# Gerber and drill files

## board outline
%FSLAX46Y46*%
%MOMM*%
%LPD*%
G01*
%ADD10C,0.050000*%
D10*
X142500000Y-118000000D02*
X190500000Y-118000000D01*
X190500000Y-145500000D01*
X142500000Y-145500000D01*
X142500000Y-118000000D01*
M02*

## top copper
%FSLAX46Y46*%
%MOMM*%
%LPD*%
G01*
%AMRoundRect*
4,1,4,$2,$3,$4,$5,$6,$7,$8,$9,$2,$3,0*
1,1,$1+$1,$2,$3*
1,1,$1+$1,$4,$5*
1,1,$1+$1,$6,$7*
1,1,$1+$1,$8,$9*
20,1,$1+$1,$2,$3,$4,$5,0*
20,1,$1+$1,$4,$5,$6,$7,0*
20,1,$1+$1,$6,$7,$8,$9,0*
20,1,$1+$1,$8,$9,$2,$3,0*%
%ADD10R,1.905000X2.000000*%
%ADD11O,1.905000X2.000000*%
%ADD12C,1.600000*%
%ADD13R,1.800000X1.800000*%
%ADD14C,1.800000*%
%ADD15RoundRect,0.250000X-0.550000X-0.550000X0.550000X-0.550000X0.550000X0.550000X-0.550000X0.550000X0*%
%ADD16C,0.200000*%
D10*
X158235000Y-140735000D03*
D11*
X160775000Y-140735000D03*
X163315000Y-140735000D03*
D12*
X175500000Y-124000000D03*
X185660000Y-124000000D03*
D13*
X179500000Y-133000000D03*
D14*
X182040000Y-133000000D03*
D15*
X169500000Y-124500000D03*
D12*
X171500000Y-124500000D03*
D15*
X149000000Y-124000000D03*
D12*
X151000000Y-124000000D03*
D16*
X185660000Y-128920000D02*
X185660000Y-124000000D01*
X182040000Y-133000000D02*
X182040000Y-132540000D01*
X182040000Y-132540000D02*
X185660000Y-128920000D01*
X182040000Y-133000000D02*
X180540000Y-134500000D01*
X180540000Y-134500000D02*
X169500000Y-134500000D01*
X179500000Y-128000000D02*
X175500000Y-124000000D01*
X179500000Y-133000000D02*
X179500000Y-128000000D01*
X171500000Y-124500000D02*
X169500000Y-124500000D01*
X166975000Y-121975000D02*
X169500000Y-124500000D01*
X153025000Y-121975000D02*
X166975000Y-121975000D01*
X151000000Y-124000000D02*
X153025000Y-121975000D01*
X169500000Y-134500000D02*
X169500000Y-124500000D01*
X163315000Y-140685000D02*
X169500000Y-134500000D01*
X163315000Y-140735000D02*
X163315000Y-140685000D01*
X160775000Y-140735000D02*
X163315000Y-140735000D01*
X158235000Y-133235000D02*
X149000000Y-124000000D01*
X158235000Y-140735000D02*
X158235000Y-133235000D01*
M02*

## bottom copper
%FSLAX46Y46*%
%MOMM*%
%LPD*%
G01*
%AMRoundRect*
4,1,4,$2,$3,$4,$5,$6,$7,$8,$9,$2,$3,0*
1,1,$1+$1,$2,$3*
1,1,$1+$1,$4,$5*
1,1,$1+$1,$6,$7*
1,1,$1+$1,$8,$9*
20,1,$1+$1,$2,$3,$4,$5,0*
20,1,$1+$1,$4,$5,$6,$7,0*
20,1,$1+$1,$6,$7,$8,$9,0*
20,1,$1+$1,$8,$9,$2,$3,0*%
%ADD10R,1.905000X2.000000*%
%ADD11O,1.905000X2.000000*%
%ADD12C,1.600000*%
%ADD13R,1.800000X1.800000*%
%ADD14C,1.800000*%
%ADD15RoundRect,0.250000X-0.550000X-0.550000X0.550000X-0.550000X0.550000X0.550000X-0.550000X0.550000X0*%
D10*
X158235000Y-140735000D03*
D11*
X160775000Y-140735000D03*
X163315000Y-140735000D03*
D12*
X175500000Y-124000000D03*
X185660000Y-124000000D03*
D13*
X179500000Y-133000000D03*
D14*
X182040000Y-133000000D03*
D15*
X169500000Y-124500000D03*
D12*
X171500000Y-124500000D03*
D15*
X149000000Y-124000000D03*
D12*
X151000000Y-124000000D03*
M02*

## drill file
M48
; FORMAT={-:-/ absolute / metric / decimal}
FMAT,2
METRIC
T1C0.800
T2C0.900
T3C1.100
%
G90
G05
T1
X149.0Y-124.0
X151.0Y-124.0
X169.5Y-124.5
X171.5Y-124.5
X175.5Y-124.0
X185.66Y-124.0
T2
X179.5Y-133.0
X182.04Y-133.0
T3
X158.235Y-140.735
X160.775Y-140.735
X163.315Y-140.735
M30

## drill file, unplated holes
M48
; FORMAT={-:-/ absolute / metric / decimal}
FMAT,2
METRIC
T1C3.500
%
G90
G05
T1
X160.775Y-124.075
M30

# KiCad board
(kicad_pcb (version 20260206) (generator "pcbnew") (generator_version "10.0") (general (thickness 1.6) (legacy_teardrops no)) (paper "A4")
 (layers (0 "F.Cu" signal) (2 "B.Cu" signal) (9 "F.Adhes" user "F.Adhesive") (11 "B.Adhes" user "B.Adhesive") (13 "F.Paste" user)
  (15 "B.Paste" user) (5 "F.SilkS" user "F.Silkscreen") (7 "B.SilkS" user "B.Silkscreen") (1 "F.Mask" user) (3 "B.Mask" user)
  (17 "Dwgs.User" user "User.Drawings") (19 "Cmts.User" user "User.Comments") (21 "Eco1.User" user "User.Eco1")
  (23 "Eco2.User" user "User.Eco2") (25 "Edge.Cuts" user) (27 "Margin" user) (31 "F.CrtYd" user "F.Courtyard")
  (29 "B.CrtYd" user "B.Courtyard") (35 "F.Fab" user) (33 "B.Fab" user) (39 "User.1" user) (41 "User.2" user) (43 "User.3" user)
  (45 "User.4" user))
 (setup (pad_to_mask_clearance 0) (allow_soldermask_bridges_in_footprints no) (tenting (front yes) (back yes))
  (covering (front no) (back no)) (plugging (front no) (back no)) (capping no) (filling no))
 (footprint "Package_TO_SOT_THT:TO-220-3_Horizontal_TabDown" (layer "F.Cu") (at 158.235 140.735)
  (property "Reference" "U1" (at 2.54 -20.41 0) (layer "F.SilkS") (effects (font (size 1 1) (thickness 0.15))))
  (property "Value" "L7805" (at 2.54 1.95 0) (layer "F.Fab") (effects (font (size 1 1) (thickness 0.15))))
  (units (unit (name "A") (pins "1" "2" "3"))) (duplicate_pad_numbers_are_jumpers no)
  (pad "" np_thru_hole circle (at 2.54 -16.66) (size 3.5 3.5) (drill 3.5) (layers "*.Cu" "*.Mask"))
  (pad "1" thru_hole rect (at 0 0) (size 1.905 2) (drill 1.1) (layers "*.Cu" "*.Mask") (remove_unused_layers no) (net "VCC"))
  (pad "2" thru_hole oval (at 2.54 0) (size 1.905 2) (drill 1.1) (layers "*.Cu" "*.Mask") (remove_unused_layers no) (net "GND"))
  (pad "3" thru_hole oval (at 5.08 0) (size 1.905 2) (drill 1.1) (layers "*.Cu" "*.Mask") (remove_unused_layers no) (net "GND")))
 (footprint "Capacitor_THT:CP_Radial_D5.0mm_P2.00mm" (layer "F.Cu") (at 149 124)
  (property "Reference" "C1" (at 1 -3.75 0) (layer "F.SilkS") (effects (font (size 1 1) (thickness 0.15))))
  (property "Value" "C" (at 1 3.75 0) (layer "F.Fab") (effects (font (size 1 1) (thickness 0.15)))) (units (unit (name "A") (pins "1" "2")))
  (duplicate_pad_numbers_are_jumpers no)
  (pad "1" thru_hole roundrect (at 0 0) (size 1.6 1.6) (drill 0.8) (layers "*.Cu" "*.Mask") (remove_unused_layers no)
   (roundrect_rratio 0.15625) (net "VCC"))
  (pad "2" thru_hole circle (at 2 0) (size 1.6 1.6) (drill 0.8) (layers "*.Cu" "*.Mask") (remove_unused_layers no) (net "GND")))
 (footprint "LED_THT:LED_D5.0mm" (layer "F.Cu") (at 179.5 133)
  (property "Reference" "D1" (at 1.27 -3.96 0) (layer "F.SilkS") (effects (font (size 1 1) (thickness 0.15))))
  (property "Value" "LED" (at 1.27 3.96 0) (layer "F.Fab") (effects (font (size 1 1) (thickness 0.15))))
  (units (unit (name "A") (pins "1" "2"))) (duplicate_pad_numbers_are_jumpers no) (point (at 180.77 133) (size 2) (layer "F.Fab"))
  (pad "1" thru_hole rect (at 0 0) (size 1.8 1.8) (drill 0.9) (layers "*.Cu" "*.Mask") (remove_unused_layers no) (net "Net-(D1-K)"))
  (pad "2" thru_hole circle (at 2.54 0) (size 1.8 1.8) (drill 0.9) (layers "*.Cu" "*.Mask") (remove_unused_layers no) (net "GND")))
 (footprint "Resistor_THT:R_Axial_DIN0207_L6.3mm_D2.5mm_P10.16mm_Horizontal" (layer "F.Cu") (at 175.5 124)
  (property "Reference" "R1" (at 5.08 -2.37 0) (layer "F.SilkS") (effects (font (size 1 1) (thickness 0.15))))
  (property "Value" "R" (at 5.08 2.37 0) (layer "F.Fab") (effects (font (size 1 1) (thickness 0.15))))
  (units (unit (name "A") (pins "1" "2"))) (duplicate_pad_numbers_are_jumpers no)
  (pad "1" thru_hole circle (at 0 0) (size 1.6 1.6) (drill 0.8) (layers "*.Cu" "*.Mask") (remove_unused_layers no) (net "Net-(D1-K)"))
  (pad "2" thru_hole circle (at 10.16 0) (size 1.6 1.6) (drill 0.8) (layers "*.Cu" "*.Mask") (remove_unused_layers no) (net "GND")))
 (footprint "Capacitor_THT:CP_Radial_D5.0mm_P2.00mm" (layer "F.Cu") (at 169.5 124.5)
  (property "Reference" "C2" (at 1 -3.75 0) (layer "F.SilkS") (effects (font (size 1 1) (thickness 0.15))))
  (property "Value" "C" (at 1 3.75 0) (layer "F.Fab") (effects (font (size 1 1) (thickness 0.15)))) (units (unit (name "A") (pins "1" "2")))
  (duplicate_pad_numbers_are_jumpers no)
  (pad "1" thru_hole roundrect (at 0 0) (size 1.6 1.6) (drill 0.8) (layers "*.Cu" "*.Mask") (remove_unused_layers no)
   (roundrect_rratio 0.15625) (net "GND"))
  (pad "2" thru_hole circle (at 2 0) (size 1.6 1.6) (drill 0.8) (layers "*.Cu" "*.Mask") (remove_unused_layers no) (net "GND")))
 (gr_rect (start 142.5 118) (end 190.5 145.5) (stroke (width 0.05) (type default)) (fill no) (layer "Edge.Cuts"))
 (segment (start 185.66 128.92) (end 185.66 124) (width 0.2) (layer "F.Cu") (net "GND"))
 (segment (start 182.04 132.54) (end 185.66 128.92) (width 0.2) (layer "F.Cu") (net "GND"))
 (segment (start 153.025 121.975) (end 166.975 121.975) (width 0.2) (layer "F.Cu") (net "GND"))
 (segment (start 163.315 140.685) (end 169.5 134.5) (width 0.2) (layer "F.Cu") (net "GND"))
 (segment (start 171.5 124.5) (end 169.5 124.5) (width 0.2) (layer "F.Cu") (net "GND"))
 (segment (start 182.04 133) (end 180.54 134.5) (width 0.2) (layer "F.Cu") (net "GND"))
 (segment (start 182.04 133) (end 182.04 132.54) (width 0.2) (layer "F.Cu") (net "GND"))
 (segment (start 166.975 121.975) (end 169.5 124.5) (width 0.2) (layer "F.Cu") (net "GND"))
 (segment (start 151 124) (end 153.025 121.975) (width 0.2) (layer "F.Cu") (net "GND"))
 (segment (start 180.54 134.5) (end 169.5 134.5) (width 0.2) (layer "F.Cu") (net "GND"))
 (segment (start 160.775 140.735) (end 163.315 140.735) (width 0.2) (layer "F.Cu") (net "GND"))
 (segment (start 169.5 134.5) (end 169.5 124.5) (width 0.2) (layer "F.Cu") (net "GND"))
 (segment (start 163.315 140.735) (end 163.315 140.685) (width 0.2) (layer "F.Cu") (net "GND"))
 (segment (start 158.235 133.235) (end 149 124) (width 0.2) (layer "F.Cu") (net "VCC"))
 (segment (start 158.235 140.735) (end 158.235 133.235) (width 0.2) (layer "F.Cu") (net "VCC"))
 (segment (start 179.5 128) (end 175.5 124) (width 0.2) (layer "F.Cu") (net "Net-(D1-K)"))
 (segment (start 179.5 133) (end 179.5 128) (width 0.2) (layer "F.Cu") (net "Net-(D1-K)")))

